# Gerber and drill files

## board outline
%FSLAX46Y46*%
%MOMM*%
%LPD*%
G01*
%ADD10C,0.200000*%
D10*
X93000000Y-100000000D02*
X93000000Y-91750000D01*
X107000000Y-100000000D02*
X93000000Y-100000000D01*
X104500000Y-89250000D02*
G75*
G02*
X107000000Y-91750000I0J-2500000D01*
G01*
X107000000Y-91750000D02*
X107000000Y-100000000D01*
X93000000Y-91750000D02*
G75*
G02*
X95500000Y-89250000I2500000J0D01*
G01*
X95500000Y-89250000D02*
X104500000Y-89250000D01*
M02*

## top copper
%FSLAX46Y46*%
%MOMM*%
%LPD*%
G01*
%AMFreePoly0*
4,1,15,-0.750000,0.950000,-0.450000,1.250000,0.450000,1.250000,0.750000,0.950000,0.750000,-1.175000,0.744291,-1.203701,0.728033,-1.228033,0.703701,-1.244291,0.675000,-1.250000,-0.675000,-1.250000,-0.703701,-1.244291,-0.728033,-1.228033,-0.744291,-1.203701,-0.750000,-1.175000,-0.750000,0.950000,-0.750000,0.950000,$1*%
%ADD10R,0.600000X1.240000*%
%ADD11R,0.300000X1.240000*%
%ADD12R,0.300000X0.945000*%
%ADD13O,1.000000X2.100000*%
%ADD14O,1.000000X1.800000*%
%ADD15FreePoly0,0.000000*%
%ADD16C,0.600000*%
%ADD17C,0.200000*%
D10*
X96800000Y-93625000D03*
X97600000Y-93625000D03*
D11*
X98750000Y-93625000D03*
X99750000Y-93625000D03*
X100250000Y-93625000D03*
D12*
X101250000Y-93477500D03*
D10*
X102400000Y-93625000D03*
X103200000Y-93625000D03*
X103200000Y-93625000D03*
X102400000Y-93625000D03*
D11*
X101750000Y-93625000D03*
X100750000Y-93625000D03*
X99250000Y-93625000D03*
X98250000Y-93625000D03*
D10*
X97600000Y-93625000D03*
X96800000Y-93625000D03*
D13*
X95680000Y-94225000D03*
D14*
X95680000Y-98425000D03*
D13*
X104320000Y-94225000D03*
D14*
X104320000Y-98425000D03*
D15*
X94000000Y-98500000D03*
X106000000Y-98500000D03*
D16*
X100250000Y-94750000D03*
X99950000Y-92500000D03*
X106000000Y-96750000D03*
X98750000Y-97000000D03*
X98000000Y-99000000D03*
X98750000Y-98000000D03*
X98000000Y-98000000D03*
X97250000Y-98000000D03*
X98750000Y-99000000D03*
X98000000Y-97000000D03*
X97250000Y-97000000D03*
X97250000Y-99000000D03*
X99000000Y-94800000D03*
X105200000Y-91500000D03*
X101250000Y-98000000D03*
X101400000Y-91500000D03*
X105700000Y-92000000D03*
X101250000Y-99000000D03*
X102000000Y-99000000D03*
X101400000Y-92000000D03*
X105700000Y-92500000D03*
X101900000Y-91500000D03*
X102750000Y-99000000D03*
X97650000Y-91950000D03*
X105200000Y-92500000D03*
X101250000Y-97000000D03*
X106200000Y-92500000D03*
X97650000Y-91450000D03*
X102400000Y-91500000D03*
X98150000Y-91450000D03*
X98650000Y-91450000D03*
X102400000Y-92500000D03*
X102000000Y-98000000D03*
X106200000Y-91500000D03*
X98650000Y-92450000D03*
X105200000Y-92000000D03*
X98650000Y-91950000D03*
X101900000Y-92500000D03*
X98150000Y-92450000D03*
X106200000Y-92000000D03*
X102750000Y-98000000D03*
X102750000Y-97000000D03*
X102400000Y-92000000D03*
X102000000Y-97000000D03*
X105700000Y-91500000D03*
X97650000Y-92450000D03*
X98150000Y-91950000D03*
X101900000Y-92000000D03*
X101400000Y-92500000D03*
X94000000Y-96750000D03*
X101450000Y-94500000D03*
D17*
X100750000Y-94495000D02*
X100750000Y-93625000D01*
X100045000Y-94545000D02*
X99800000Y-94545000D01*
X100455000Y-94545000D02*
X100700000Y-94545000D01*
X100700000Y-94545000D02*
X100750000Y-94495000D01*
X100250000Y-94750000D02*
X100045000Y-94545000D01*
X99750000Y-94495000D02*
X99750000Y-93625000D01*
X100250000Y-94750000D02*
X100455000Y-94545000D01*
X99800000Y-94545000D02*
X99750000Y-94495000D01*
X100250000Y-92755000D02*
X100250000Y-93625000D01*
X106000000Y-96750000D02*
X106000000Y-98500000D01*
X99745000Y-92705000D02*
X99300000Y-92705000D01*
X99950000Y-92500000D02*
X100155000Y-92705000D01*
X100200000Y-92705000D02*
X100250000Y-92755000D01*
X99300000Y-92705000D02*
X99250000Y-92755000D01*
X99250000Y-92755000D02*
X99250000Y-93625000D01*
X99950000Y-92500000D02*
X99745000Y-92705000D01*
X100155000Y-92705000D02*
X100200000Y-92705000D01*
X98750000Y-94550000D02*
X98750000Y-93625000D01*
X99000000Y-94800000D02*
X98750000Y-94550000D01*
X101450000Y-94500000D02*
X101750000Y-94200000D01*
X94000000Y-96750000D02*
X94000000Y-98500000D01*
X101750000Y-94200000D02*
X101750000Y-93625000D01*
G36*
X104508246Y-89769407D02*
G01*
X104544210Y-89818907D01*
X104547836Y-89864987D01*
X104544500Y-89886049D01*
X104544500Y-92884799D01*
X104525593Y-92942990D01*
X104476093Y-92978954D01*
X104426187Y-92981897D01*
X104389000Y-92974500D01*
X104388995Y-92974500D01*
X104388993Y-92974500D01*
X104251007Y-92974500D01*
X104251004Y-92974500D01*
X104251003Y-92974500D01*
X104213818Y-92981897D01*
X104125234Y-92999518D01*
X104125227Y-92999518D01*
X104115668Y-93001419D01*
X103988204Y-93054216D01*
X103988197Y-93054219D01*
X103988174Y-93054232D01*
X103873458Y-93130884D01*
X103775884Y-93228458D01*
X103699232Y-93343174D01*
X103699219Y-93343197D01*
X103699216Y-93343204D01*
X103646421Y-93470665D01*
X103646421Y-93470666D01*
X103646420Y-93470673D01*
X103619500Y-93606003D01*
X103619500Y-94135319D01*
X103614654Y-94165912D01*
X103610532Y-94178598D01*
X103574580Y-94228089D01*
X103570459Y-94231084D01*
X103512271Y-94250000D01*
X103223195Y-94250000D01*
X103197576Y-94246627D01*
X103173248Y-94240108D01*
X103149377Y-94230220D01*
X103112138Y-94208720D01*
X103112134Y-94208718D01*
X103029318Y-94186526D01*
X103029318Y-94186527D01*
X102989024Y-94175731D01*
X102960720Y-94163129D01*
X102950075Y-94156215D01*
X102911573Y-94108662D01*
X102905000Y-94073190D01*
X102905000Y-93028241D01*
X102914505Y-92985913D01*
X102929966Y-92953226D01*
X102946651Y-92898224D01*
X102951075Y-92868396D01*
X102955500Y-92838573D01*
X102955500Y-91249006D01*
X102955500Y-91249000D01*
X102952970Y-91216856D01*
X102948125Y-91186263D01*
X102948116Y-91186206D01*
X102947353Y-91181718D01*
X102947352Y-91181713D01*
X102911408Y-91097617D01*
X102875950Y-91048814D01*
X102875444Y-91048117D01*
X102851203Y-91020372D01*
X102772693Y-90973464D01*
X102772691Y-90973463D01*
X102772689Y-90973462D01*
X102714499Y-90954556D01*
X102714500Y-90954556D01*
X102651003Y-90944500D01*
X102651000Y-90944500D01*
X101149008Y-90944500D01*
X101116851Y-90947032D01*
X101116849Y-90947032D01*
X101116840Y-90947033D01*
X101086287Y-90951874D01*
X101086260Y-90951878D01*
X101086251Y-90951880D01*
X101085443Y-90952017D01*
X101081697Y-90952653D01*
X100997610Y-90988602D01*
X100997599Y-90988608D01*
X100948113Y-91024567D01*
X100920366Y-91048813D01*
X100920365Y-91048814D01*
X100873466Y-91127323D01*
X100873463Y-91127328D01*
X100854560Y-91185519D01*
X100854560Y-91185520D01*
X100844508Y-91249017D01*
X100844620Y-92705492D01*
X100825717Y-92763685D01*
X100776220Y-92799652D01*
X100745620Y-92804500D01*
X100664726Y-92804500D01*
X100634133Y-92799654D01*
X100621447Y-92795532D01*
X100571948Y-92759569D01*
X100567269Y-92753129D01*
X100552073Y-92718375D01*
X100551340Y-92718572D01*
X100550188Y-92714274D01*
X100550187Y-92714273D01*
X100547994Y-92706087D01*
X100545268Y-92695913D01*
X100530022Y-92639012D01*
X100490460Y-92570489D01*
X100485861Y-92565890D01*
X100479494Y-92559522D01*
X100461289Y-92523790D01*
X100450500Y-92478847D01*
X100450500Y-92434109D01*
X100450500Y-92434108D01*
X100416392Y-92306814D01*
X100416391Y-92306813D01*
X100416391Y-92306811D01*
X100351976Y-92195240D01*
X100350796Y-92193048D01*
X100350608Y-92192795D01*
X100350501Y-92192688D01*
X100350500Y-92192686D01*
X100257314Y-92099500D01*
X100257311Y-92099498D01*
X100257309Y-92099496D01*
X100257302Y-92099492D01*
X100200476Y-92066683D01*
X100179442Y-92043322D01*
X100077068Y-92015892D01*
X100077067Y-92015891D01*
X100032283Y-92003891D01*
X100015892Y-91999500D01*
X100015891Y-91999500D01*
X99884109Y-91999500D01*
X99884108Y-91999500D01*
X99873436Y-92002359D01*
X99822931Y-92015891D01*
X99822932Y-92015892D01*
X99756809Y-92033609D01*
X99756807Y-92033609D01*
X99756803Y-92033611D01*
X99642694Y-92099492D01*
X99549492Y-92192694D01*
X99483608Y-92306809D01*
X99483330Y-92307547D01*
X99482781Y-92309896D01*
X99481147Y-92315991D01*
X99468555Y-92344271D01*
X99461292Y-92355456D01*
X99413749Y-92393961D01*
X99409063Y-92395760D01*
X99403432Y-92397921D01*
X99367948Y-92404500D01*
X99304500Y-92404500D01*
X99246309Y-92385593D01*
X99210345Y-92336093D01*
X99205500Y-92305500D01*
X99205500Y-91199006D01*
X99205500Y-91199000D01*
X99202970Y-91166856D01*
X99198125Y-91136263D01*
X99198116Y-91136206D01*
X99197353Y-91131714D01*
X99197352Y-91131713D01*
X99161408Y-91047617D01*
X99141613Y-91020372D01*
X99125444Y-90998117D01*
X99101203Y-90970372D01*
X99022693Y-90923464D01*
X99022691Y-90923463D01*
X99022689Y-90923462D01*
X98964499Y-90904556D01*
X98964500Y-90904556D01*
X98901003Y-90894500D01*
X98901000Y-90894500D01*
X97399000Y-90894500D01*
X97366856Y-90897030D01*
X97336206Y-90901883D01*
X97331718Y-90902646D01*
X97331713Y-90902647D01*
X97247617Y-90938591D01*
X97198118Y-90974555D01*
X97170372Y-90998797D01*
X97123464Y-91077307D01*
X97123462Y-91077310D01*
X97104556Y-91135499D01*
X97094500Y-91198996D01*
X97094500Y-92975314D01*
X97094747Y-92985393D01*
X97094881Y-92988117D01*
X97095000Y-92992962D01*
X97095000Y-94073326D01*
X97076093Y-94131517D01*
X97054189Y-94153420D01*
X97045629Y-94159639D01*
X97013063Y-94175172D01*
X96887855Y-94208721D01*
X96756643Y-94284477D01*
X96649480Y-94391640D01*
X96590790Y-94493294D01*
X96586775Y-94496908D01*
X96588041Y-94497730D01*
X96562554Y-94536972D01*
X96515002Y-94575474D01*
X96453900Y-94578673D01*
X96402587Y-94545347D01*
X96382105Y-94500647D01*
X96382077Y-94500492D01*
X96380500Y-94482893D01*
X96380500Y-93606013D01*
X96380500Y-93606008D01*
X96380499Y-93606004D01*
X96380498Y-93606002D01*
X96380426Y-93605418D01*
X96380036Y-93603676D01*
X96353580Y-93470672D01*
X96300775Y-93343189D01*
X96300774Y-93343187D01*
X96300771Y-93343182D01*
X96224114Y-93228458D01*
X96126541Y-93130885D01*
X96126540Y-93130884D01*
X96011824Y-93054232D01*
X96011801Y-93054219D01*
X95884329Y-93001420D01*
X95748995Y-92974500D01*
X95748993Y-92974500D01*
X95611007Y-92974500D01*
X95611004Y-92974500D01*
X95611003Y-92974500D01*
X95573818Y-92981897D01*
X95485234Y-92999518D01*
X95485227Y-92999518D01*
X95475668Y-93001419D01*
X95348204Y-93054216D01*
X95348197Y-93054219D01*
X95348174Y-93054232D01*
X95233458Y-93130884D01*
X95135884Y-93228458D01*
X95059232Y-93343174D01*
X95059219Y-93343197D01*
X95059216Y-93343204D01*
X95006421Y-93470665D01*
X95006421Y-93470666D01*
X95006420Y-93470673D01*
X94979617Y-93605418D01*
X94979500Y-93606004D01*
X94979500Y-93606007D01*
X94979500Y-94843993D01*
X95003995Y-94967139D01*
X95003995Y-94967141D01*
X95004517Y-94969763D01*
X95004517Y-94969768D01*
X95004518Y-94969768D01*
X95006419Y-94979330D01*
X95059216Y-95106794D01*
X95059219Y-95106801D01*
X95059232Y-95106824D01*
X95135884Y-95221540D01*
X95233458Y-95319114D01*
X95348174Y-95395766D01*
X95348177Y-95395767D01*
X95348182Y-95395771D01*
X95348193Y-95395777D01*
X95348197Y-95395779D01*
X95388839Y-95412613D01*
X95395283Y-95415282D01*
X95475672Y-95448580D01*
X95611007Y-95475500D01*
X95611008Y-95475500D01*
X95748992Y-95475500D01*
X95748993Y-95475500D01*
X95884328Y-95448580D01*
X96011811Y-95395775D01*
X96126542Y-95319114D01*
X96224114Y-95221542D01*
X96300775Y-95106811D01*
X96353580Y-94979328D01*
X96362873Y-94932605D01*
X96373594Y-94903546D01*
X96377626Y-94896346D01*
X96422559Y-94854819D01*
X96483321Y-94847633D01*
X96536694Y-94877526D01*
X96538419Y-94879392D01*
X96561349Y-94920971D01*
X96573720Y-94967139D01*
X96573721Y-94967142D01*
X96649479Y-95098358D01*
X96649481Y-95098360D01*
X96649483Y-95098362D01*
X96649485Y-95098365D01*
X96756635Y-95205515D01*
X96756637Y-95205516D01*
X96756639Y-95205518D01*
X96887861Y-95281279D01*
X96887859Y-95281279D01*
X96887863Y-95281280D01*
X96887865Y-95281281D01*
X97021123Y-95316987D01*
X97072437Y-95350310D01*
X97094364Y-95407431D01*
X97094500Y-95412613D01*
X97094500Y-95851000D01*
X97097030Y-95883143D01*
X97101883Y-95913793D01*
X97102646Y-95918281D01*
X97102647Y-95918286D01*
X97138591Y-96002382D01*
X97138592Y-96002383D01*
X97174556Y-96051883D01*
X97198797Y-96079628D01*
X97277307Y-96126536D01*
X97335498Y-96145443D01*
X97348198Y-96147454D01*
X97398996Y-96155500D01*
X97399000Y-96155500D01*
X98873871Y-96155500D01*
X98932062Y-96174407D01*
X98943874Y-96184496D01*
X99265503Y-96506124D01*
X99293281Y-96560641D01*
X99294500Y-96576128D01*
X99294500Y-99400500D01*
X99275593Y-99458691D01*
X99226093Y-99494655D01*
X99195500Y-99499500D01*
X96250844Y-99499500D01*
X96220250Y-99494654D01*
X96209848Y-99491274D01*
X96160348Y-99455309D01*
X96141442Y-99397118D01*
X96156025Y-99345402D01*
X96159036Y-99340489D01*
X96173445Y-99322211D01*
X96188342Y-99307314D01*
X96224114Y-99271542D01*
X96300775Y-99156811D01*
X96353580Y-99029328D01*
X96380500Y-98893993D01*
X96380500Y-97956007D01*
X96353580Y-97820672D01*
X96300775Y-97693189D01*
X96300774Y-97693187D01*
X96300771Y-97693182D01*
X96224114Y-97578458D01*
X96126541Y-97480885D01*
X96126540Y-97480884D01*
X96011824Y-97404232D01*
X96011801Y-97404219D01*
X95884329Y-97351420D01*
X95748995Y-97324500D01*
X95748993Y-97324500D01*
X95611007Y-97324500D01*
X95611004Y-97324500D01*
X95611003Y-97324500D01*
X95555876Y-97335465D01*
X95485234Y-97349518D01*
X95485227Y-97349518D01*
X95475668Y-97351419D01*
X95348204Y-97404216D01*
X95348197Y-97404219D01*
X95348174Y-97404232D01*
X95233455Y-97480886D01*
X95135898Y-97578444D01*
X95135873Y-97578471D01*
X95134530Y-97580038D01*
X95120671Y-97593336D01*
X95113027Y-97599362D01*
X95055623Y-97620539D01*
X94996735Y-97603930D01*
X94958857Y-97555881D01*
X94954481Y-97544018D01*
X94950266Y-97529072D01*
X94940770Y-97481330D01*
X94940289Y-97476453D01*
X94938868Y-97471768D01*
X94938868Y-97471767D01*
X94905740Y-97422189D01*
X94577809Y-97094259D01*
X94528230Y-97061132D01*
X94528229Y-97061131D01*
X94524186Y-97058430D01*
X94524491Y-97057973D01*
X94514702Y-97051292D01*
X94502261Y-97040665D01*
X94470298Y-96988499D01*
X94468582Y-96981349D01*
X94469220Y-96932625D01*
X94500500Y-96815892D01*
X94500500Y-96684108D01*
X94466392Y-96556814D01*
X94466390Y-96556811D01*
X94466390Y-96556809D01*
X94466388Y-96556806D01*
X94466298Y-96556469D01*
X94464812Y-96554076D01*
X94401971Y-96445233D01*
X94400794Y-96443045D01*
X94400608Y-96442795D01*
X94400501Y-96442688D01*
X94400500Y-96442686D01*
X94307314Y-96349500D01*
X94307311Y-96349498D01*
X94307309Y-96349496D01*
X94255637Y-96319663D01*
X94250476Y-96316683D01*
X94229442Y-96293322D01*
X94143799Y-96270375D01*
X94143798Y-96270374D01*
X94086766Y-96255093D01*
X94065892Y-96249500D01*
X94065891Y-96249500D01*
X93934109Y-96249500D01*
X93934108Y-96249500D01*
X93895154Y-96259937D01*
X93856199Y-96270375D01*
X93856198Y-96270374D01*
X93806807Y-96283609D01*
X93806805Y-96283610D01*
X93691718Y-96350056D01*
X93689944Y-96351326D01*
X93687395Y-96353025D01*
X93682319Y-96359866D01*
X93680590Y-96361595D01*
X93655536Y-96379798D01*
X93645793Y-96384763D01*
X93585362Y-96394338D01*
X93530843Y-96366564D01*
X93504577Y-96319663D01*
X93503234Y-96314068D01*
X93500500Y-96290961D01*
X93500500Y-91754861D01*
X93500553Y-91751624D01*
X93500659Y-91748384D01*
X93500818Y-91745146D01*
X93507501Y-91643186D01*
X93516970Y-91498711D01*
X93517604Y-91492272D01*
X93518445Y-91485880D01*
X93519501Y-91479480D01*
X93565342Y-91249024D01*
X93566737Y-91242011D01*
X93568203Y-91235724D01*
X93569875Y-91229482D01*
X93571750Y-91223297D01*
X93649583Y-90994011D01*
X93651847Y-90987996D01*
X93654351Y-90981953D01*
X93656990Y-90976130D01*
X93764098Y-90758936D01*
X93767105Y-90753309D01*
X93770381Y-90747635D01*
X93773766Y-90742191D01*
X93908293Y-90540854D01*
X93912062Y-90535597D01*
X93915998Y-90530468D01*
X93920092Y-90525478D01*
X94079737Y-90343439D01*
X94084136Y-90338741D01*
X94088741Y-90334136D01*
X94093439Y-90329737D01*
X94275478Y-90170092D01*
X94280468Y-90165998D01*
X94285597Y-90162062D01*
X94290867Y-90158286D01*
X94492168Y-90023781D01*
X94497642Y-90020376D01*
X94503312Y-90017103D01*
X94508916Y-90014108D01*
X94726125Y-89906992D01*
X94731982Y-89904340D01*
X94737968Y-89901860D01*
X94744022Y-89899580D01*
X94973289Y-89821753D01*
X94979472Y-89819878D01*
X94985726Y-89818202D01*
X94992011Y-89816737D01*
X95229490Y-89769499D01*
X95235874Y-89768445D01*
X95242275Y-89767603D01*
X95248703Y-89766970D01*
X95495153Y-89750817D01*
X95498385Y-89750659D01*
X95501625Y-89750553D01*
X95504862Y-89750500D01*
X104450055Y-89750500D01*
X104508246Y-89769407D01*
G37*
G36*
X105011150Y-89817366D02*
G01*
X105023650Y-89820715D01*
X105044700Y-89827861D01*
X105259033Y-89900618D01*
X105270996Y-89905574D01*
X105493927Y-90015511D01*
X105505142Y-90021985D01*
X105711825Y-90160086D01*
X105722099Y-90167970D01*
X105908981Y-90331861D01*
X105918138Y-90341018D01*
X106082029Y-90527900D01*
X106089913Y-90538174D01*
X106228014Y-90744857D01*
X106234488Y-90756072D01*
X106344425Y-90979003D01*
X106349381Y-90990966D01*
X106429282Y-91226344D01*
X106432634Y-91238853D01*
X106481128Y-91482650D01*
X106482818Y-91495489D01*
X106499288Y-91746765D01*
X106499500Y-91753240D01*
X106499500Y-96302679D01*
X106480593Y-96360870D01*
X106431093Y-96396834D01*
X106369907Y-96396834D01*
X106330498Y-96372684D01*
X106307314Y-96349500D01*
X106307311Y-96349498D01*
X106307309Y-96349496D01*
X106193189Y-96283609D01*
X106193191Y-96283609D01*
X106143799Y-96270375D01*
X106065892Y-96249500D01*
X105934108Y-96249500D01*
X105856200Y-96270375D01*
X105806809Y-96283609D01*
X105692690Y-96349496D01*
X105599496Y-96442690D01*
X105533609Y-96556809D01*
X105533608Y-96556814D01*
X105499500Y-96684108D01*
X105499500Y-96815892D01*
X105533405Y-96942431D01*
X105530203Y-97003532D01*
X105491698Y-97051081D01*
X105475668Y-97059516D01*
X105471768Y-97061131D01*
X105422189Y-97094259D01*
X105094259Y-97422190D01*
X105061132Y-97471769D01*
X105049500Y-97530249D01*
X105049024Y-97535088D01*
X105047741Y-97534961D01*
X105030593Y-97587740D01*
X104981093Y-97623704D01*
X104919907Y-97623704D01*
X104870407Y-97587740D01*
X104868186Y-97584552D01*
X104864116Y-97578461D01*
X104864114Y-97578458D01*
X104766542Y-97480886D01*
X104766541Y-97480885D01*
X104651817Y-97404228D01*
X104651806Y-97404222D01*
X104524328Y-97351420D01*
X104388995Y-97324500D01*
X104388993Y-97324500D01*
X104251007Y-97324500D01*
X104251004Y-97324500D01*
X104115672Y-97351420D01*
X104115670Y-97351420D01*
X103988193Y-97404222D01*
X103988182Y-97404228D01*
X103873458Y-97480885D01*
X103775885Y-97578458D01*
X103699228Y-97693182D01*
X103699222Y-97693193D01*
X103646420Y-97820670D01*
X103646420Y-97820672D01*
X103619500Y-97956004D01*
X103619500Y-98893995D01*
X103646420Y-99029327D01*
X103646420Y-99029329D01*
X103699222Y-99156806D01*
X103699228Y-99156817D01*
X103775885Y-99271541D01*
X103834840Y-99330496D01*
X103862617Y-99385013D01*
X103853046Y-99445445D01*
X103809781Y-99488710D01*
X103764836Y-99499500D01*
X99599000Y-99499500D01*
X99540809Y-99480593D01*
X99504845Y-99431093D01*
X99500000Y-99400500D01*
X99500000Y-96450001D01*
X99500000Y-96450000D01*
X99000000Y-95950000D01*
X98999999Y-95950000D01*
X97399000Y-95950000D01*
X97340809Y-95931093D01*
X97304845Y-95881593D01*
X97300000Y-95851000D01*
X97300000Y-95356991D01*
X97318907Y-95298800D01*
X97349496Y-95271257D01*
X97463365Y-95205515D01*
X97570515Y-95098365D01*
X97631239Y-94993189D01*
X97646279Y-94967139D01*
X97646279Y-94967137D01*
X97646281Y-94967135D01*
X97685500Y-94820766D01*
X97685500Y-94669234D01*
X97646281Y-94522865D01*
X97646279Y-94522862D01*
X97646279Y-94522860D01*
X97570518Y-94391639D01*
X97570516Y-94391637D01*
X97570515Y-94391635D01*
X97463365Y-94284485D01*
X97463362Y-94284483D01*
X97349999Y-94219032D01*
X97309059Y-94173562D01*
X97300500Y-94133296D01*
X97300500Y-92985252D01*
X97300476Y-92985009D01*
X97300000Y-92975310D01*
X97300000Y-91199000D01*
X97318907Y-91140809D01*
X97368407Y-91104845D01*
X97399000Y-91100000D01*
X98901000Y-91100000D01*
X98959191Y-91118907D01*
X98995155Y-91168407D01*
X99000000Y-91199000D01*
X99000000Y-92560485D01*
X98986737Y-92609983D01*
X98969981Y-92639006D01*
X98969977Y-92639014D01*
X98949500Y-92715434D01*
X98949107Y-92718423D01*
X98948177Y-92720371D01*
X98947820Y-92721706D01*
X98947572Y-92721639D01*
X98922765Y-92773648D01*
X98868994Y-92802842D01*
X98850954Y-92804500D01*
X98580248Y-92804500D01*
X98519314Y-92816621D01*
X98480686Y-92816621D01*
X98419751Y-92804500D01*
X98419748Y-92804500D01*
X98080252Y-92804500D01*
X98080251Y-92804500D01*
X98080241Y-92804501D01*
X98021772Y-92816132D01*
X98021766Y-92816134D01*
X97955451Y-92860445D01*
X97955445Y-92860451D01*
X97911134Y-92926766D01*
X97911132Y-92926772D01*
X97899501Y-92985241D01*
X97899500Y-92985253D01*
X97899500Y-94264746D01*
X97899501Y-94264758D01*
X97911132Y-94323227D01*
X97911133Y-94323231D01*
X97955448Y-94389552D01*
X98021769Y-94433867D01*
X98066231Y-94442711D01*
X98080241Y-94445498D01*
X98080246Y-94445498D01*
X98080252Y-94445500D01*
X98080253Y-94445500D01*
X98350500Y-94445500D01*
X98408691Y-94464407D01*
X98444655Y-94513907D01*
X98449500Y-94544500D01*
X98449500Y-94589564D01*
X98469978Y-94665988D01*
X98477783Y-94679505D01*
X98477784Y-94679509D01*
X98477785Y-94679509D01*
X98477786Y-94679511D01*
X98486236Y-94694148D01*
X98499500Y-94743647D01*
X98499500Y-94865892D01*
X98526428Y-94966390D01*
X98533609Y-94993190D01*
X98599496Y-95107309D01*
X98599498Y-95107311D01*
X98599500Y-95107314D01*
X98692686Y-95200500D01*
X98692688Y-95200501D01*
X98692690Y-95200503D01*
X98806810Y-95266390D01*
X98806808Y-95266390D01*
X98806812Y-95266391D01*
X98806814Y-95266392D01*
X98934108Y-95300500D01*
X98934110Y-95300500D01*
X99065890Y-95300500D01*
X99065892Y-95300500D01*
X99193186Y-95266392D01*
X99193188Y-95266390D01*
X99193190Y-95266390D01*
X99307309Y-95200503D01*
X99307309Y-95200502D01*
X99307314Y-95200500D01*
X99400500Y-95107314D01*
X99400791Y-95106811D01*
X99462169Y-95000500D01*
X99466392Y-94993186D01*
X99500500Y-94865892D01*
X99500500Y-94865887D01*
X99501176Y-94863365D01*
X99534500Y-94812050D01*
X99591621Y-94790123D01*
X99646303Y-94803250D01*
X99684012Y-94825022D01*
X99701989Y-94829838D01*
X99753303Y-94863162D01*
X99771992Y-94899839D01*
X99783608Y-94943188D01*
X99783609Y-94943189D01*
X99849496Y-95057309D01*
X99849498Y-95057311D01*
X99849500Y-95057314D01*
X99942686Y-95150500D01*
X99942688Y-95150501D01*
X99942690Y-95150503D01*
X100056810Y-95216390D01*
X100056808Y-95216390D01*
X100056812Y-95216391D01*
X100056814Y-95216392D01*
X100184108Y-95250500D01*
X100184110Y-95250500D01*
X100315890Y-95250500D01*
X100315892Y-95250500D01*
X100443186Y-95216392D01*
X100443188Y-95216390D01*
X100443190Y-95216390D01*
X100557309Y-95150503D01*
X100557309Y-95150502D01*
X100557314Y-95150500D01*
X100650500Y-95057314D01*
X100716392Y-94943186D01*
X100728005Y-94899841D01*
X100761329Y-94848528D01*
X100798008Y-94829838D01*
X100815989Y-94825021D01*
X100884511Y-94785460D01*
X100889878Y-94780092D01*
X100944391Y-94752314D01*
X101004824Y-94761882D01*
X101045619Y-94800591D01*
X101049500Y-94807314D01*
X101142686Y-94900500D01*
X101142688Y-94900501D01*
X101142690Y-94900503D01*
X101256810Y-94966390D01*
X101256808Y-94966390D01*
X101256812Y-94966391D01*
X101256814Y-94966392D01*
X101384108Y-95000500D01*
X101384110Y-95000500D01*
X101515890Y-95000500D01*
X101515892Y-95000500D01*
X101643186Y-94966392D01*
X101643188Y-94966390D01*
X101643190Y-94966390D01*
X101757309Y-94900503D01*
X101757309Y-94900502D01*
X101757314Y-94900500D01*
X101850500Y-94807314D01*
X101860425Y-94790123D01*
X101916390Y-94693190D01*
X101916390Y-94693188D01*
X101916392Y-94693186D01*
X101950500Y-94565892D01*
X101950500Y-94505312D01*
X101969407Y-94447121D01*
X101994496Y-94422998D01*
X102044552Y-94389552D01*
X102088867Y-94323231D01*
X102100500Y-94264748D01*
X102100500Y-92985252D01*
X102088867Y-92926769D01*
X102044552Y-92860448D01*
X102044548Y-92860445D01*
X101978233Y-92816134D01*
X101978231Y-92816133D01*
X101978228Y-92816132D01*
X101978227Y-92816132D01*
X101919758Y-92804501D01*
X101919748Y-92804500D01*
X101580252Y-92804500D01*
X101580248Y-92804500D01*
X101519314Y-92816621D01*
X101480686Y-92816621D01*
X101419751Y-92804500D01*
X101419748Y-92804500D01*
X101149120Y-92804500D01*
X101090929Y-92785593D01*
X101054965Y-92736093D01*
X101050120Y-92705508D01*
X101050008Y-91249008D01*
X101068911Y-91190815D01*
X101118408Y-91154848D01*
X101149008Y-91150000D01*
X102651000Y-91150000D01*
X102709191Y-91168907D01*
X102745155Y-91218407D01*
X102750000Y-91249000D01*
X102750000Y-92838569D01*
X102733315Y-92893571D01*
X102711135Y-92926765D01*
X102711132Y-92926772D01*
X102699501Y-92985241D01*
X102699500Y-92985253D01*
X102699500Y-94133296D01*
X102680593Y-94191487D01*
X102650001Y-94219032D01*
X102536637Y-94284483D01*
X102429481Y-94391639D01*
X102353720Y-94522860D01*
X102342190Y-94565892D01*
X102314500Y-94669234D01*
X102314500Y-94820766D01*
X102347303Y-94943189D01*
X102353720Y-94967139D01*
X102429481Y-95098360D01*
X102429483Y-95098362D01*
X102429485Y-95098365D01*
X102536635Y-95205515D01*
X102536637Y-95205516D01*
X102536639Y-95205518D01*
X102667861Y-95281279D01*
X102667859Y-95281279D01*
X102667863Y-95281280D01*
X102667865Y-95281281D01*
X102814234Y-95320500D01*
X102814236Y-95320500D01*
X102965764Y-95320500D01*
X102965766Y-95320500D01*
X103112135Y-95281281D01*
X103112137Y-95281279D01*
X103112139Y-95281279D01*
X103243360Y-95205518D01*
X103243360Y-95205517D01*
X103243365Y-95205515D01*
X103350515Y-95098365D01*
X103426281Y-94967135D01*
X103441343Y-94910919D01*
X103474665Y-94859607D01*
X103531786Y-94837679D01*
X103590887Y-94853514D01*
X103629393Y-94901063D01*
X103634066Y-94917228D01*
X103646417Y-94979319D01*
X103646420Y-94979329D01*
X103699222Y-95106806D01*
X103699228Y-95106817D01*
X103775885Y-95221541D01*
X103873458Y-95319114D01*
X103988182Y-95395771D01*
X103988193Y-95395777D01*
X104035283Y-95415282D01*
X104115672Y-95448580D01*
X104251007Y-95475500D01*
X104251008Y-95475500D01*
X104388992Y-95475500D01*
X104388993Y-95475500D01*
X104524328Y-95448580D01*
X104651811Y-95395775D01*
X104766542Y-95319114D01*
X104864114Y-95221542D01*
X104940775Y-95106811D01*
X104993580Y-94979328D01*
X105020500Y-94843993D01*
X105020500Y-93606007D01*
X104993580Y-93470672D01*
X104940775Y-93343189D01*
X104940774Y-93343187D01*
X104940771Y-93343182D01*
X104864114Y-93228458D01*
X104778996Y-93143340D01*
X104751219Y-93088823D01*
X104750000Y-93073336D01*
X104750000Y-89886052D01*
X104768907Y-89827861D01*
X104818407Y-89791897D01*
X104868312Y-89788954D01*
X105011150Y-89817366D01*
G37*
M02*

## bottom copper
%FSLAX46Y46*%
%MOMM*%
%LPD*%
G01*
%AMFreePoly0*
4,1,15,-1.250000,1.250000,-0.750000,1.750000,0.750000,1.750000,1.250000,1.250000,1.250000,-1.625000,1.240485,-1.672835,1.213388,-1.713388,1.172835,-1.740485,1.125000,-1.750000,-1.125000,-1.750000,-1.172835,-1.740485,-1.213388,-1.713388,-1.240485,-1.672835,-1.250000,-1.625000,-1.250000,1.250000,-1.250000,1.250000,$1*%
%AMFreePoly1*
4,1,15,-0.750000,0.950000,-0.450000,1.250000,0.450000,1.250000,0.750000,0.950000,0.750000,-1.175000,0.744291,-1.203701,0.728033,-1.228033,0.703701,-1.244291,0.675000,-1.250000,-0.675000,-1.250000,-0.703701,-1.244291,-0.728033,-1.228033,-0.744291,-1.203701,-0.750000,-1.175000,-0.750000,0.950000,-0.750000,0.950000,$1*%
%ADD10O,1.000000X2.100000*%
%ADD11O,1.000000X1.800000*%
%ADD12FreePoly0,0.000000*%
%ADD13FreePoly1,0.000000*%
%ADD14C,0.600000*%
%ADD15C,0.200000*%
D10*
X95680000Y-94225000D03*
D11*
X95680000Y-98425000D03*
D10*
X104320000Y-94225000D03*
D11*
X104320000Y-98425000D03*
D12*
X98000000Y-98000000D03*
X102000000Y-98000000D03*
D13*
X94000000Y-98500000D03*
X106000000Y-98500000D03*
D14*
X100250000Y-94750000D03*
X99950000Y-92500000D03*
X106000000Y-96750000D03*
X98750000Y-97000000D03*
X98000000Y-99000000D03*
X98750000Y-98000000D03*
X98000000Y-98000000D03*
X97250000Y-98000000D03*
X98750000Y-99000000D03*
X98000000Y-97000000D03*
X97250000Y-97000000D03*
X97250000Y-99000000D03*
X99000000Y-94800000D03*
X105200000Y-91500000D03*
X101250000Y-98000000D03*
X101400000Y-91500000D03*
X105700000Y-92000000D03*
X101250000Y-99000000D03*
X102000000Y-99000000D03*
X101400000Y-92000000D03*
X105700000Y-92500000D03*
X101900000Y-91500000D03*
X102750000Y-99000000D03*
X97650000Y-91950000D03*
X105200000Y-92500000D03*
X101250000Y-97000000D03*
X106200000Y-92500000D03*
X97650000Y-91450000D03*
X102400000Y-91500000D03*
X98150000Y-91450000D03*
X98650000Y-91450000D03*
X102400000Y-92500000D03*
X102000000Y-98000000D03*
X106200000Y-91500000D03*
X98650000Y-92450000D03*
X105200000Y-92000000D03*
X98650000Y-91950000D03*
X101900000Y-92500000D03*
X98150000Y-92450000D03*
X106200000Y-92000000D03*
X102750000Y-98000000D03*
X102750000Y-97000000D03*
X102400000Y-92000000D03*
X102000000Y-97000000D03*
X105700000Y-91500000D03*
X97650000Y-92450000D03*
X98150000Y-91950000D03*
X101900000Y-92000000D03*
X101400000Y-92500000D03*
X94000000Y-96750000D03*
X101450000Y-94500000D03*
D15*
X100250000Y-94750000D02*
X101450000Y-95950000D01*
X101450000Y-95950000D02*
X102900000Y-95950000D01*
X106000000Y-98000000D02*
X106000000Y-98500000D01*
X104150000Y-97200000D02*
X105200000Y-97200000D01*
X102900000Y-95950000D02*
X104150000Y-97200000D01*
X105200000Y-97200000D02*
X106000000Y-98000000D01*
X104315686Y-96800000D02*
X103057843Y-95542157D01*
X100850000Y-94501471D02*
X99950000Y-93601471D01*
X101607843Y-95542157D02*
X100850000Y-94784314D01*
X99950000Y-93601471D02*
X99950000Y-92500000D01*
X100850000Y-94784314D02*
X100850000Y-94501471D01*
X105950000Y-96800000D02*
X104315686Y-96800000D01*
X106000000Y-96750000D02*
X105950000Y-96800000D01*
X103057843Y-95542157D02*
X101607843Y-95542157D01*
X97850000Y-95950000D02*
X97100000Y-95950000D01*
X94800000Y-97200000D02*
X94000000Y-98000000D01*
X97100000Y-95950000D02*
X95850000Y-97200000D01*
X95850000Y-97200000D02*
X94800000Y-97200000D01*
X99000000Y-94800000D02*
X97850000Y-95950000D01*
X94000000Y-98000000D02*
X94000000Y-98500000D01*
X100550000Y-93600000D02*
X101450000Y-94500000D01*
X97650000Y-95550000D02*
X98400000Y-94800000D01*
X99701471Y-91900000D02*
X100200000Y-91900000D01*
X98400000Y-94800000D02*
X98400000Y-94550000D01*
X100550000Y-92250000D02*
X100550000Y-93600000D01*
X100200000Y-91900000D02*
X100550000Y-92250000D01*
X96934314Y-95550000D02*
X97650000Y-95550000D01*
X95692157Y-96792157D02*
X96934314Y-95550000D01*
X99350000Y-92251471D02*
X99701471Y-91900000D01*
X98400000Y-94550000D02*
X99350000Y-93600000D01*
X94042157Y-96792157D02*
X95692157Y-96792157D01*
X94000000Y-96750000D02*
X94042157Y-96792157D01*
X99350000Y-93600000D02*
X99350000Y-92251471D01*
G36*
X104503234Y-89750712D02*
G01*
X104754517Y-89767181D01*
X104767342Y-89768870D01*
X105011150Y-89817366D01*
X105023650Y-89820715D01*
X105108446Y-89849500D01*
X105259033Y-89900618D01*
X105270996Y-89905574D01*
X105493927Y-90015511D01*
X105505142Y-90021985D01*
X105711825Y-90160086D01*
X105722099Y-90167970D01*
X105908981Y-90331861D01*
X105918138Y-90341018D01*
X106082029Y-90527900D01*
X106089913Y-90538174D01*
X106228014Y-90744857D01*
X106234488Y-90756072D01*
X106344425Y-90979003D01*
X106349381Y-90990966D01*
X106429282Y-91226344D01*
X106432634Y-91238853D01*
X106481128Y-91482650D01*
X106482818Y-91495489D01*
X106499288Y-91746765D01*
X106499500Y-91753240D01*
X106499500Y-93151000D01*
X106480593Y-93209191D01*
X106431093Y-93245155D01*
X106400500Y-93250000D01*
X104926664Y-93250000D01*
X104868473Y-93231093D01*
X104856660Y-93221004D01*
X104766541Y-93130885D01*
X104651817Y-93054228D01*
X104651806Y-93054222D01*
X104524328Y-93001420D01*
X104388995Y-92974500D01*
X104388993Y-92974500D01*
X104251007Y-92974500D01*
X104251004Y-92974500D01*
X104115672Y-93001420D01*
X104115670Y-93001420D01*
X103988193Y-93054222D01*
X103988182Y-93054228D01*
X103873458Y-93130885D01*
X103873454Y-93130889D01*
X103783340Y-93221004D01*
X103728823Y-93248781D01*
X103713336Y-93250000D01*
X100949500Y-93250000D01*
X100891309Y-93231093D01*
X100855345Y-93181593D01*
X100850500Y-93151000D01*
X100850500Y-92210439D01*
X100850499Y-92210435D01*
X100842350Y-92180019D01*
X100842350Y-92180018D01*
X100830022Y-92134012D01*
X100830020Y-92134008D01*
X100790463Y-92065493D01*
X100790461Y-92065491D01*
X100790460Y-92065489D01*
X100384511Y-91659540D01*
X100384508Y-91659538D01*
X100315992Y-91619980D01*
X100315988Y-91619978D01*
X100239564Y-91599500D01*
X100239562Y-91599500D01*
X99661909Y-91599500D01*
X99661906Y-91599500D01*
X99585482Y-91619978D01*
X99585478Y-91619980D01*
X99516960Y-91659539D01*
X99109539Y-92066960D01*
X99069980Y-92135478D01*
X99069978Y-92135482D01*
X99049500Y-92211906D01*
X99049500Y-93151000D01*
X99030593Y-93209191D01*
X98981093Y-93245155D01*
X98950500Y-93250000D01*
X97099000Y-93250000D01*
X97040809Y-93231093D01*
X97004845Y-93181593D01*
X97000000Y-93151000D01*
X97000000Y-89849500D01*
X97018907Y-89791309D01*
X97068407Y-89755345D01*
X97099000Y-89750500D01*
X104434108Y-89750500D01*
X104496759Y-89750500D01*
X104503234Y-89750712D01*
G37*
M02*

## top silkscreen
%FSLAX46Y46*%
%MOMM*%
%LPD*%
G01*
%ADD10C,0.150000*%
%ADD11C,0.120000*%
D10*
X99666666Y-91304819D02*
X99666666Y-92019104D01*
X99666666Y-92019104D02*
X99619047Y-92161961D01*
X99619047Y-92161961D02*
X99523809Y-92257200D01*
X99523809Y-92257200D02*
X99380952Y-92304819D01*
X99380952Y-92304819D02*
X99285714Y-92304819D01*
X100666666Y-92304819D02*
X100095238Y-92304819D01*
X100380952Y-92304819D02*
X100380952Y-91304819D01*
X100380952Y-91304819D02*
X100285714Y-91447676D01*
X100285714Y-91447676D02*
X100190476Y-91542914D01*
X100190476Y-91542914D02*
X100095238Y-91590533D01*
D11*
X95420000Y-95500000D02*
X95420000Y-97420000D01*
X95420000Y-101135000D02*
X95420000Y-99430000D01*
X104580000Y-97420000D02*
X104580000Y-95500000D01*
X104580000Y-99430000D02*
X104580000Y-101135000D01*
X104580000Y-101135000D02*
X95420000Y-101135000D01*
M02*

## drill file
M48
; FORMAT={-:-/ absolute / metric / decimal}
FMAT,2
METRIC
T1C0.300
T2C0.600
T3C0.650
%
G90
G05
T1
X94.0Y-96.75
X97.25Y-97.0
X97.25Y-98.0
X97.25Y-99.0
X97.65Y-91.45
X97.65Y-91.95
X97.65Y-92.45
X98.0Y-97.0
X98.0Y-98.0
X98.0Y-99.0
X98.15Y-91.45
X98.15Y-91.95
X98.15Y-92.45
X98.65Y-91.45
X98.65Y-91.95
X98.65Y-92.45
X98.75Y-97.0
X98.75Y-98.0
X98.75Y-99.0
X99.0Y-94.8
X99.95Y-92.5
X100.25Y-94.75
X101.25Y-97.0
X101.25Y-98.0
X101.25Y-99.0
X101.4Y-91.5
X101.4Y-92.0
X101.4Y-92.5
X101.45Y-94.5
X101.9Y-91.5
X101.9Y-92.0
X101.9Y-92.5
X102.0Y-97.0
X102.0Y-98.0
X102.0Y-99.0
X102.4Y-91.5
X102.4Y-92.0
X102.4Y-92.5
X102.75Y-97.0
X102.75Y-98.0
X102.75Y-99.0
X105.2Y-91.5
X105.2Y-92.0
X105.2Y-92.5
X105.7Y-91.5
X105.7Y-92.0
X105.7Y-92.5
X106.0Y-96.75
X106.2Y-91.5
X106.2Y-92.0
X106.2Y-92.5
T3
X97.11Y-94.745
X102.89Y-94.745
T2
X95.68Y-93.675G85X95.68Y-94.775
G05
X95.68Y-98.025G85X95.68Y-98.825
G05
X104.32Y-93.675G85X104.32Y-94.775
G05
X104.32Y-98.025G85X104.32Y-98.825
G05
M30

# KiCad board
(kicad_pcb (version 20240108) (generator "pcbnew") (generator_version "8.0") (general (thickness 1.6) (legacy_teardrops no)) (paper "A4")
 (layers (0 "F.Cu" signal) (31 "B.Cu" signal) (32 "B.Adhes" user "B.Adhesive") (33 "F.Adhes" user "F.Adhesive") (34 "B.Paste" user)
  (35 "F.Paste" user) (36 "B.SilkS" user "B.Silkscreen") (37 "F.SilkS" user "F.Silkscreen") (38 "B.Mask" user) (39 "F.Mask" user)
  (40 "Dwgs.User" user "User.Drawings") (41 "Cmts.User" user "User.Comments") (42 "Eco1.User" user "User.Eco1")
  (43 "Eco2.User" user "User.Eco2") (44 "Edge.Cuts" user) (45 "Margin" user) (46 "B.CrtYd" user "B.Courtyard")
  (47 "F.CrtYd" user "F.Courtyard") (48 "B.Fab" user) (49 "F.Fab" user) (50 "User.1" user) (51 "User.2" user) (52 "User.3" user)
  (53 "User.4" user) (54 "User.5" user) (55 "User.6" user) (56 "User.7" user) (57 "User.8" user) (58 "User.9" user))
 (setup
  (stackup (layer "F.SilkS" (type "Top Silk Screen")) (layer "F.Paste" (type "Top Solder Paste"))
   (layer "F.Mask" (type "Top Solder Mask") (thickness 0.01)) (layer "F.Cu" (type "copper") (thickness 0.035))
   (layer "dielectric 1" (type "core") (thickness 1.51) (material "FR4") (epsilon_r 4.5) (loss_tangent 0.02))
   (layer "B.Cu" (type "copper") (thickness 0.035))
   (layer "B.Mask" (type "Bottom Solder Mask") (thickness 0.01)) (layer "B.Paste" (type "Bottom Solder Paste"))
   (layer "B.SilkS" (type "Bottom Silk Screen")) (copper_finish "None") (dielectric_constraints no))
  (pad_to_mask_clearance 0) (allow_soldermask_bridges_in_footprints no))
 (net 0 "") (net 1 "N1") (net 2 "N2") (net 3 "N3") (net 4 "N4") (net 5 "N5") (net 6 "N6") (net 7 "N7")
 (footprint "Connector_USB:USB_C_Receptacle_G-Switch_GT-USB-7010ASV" (layer "F.Cu") (at 100 97.35)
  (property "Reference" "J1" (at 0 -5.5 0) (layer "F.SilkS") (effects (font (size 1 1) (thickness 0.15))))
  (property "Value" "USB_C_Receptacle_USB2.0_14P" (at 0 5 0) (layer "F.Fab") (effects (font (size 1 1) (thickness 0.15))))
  (fp_line (start -4.58 -1.85) (end -4.58 0.07) (stroke (width 0.12) (type solid)) (layer "F.SilkS"))
  (fp_line (start -4.58 3.785) (end -4.58 2.08) (stroke (width 0.12) (type solid)) (layer "F.SilkS"))
  (fp_line (start 4.58 0.07) (end 4.58 -1.85) (stroke (width 0.12) (type solid)) (layer "F.SilkS"))
  (fp_line (start 4.58 2.08) (end 4.58 3.785) (stroke (width 0.12) (type solid)) (layer "F.SilkS"))
  (fp_line (start 4.58 3.785) (end -4.58 3.785) (stroke (width 0.12) (type solid)) (layer "F.SilkS"))
  (pad "" np_thru_hole circle (at -2.89 -2.605) (size 0.65 0.65) (drill 0.65) (layers "*.Cu" "*.Mask"))
  (pad "" np_thru_hole circle (at 2.89 -2.605) (size 0.65 0.65) (drill 0.65) (layers "*.Cu" "*.Mask"))
  (pad "A1" smd rect (at -3.2 -3.725) (size 0.6 1.24) (layers "F.Cu" "F.Paste" "F.Mask") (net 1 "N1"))
  (pad "A4" smd rect (at -2.4 -3.725) (size 0.6 1.24) (layers "F.Cu" "F.Paste" "F.Mask") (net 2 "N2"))
  (pad "A5" smd rect (at -1.25 -3.725) (size 0.3 1.24) (layers "F.Cu" "F.Paste" "F.Mask") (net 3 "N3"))
  (pad "A6" smd rect (at -0.25 -3.725) (size 0.3 1.24) (layers "F.Cu" "F.Paste" "F.Mask") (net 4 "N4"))
  (pad "A7" smd rect (at 0.25 -3.725) (size 0.3 1.24) (layers "F.Cu" "F.Paste" "F.Mask") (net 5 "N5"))
  (pad "A8" smd rect (at 1.25 -3.8725) (size 0.3 0.945) (layers "F.Cu" "F.Paste" "F.Mask"))
  (pad "A9" smd rect (at 2.4 -3.725) (size 0.6 1.24) (layers "F.Cu" "F.Paste" "F.Mask") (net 2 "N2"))
  (pad "A12" smd rect (at 3.2 -3.725) (size 0.6 1.24) (layers "F.Cu" "F.Paste" "F.Mask") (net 1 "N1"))
  (pad "B1" smd rect (at 3.2 -3.725) (size 0.6 1.24) (layers "F.Cu" "F.Paste" "F.Mask") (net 1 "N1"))
  (pad "B4" smd rect (at 2.4 -3.725) (size 0.6 1.24) (layers "F.Cu" "F.Paste" "F.Mask") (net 2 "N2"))
  (pad "B5" smd rect (at 1.75 -3.725) (size 0.3 1.24) (layers "F.Cu" "F.Paste" "F.Mask") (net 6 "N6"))
  (pad "B6" smd rect (at 0.75 -3.725) (size 0.3 1.24) (layers "F.Cu" "F.Paste" "F.Mask") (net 4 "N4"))
  (pad "B7" smd rect (at -0.75 -3.725) (size 0.3 1.24) (layers "F.Cu" "F.Paste" "F.Mask") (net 5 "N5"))
  (pad "B8" smd rect (at -1.75 -3.725) (size 0.3 1.24) (layers "F.Cu" "F.Paste" "F.Mask"))
  (pad "B9" smd rect (at -2.4 -3.725) (size 0.6 1.24) (layers "F.Cu" "F.Paste" "F.Mask") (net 2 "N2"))
  (pad "B12" smd rect (at -3.2 -3.725) (size 0.6 1.24) (layers "F.Cu" "F.Paste" "F.Mask") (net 1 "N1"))
  (pad "S1" thru_hole oval (at -4.32 -3.125) (size 1 2.1) (drill oval 0.6 1.7) (layers "*.Cu" "*.Mask") (remove_unused_layers no)
   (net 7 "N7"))
  (pad "S1" thru_hole oval (at -4.32 1.075) (size 1 1.8) (drill oval 0.6 1.4) (layers "*.Cu" "*.Mask") (remove_unused_layers no)
   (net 7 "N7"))
  (pad "S1" thru_hole oval (at 4.32 -3.125) (size 1 2.1) (drill oval 0.6 1.7) (layers "*.Cu" "*.Mask") (remove_unused_layers no)
   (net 7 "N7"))
  (pad "S1" thru_hole oval (at 4.32 1.075) (size 1 1.8) (drill oval 0.6 1.4) (layers "*.Cu" "*.Mask") (remove_unused_layers no) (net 7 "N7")))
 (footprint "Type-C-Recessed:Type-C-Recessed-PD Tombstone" (layer "F.Cu") (at 100 100)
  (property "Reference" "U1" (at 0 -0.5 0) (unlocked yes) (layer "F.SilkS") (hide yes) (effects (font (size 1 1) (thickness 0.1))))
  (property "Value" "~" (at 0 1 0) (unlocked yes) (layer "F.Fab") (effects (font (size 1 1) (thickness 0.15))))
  (pad "1" smd roundrect (at -2 -2) (size 2.5 3.5) (layers "B.Cu" "B.Mask") (roundrect_rratio 0.05) (chamfer_ratio 0.2)
   (chamfer top_left top_right) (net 1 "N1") (thermal_bridge_angle 45))
  (pad "2" smd roundrect (at 2 -2) (size 2.5 3.5) (layers "B.Cu" "B.Mask") (roundrect_rratio 0.05) (chamfer_ratio 0.2)
   (chamfer top_left top_right) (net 2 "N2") (thermal_bridge_angle 45))
  (pad "3" smd roundrect (at -6 -1.5) (size 1.5 2.5) (layers "B.Cu" "B.Mask") (roundrect_rratio 0.05) (chamfer_ratio 0.2)
   (chamfer top_left top_right) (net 3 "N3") (thermal_bridge_angle 45))
  (pad "4" smd roundrect (at -6 -1.5) (size 1.5 2.5) (layers "F.Cu" "F.Mask") (roundrect_rratio 0.05) (chamfer_ratio 0.2)
   (chamfer top_left top_right) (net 6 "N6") (thermal_bridge_angle 45))
  (pad "5" smd roundrect (at 6 -1.5) (size 1.5 2.5) (layers "B.Cu" "B.Mask") (roundrect_rratio 0.05) (chamfer_ratio 0.2)
   (chamfer top_left top_right) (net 4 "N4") (thermal_bridge_angle 45))
  (pad "6" smd roundrect (at 6 -1.5) (size 1.5 2.5) (layers "F.Cu" "F.Mask") (roundrect_rratio 0.05) (chamfer_ratio 0.2)
   (chamfer top_left top_right) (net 5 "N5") (thermal_bridge_angle 45)))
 (gr_line (start 93 100) (end 93 91.75) (stroke (width 0.2) (type default)) (layer "Edge.Cuts"))
 (gr_line (start 107 100) (end 93 100) (stroke (width 0.2) (type default)) (layer "Edge.Cuts"))
 (gr_arc (start 104.5 89.25) (mid 106.267767 89.982233) (end 107 91.75) (stroke (width 0.2) (type default)) (layer "Edge.Cuts"))
 (gr_line (start 107 91.75) (end 107 100) (stroke (width 0.2) (type default)) (layer "Edge.Cuts"))
 (gr_arc (start 93 91.75) (mid 93.732233 89.982233) (end 95.5 89.25) (stroke (width 0.2) (type default)) (layer "Edge.Cuts"))
 (gr_line (start 95.5 89.25) (end 104.5 89.25) (stroke (width 0.2) (type default)) (layer "Edge.Cuts"))
 (segment (start 100.75 94.495) (end 100.75 93.625) (width 0.2) (layer "F.Cu") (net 4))
 (segment (start 100.045 94.545) (end 99.8 94.545) (width 0.2) (layer "F.Cu") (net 4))
 (segment (start 100.455 94.545) (end 100.7 94.545) (width 0.2) (layer "F.Cu") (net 4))
 (segment (start 100.7 94.545) (end 100.75 94.495) (width 0.2) (layer "F.Cu") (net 4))
 (segment (start 100.25 94.75) (end 100.045 94.545) (width 0.2) (layer "F.Cu") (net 4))
 (segment (start 99.75 94.495) (end 99.75 93.625) (width 0.2) (layer "F.Cu") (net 4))
 (segment (start 100.25 94.75) (end 100.455 94.545) (width 0.2) (layer "F.Cu") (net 4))
 (segment (start 99.8 94.545) (end 99.75 94.495) (width 0.2) (layer "F.Cu") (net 4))
 (via (at 100.25 94.75) (size 0.6) (drill 0.3) (layers "F.Cu" "B.Cu") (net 4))
 (segment (start 100.25 94.75) (end 101.45 95.95) (width 0.2) (layer "B.Cu") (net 4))
 (segment (start 101.45 95.95) (end 102.9 95.95) (width 0.2) (layer "B.Cu") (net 4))
 (segment (start 106 98) (end 106 98.5) (width 0.2) (layer "B.Cu") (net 4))
 (segment (start 104.15 97.2) (end 105.2 97.2) (width 0.2) (layer "B.Cu") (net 4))
 (segment (start 102.9 95.95) (end 104.15 97.2) (width 0.2) (layer "B.Cu") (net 4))
 (segment (start 105.2 97.2) (end 106 98) (width 0.2) (layer "B.Cu") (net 4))
 (segment (start 100.25 92.755) (end 100.25 93.625) (width 0.2) (layer "F.Cu") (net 5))
 (segment (start 106 96.75) (end 106 98.5) (width 0.2) (layer "F.Cu") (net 5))
 (segment (start 99.745 92.705) (end 99.3 92.705) (width 0.2) (layer "F.Cu") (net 5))
 (segment (start 99.95 92.5) (end 100.155 92.705) (width 0.2) (layer "F.Cu") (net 5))
 (segment (start 100.2 92.705) (end 100.25 92.755) (width 0.2) (layer "F.Cu") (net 5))
 (segment (start 99.3 92.705) (end 99.25 92.755) (width 0.2) (layer "F.Cu") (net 5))
 (segment (start 99.25 92.755) (end 99.25 93.625) (width 0.2) (layer "F.Cu") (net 5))
 (segment (start 99.95 92.5) (end 99.745 92.705) (width 0.2) (layer "F.Cu") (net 5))
 (segment (start 100.155 92.705) (end 100.2 92.705) (width 0.2) (layer "F.Cu") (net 5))
 (via (at 99.95 92.5) (size 0.6) (drill 0.3) (layers "F.Cu" "B.Cu") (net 5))
 (via (at 106 96.75) (size 0.6) (drill 0.3) (layers "F.Cu" "B.Cu") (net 5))
 (segment (start 104.315686 96.8) (end 103.057843 95.542157) (width 0.2) (layer "B.Cu") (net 5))
 (segment (start 100.85 94.501471) (end 99.95 93.601471) (width 0.2) (layer "B.Cu") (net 5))
 (segment (start 101.607843 95.542157) (end 100.85 94.784314) (width 0.2) (layer "B.Cu") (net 5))
 (segment (start 99.95 93.601471) (end 99.95 92.5) (width 0.2) (layer "B.Cu") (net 5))
 (segment (start 100.85 94.784314) (end 100.85 94.501471) (width 0.2) (layer "B.Cu") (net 5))
 (segment (start 105.95 96.8) (end 104.315686 96.8) (width 0.2) (layer "B.Cu") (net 5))
 (segment (start 106 96.75) (end 105.95 96.8) (width 0.2) (layer "B.Cu") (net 5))
 (segment (start 103.057843 95.542157) (end 101.607843 95.542157) (width 0.2) (layer "B.Cu") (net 5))
 (via (at 98.75 97) (size 0.6) (drill 0.3) (layers "F.Cu" "B.Cu") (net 1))
 (via (at 98 99) (size 0.6) (drill 0.3) (layers "F.Cu" "B.Cu") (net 1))
 (via (at 98.75 98) (size 0.6) (drill 0.3) (layers "F.Cu" "B.Cu") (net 1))
 (via (at 98 98) (size 0.6) (drill 0.3) (layers "F.Cu" "B.Cu") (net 1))
 (via (at 97.25 98) (size 0.6) (drill 0.3) (layers "F.Cu" "B.Cu") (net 1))
 (via (at 98.75 99) (size 0.6) (drill 0.3) (layers "F.Cu" "B.Cu") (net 1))
 (via (at 98 97) (size 0.6) (drill 0.3) (layers "F.Cu" "B.Cu") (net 1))
 (via (at 97.25 97) (size 0.6) (drill 0.3) (layers "F.Cu" "B.Cu") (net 1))
 (via (at 97.25 99) (size 0.6) (drill 0.3) (layers "F.Cu" "B.Cu") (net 1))
 (segment (start 98.75 94.55) (end 98.75 93.625) (width 0.2) (layer "F.Cu") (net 3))
 (segment (start 99 94.8) (end 98.75 94.55) (width 0.2) (layer "F.Cu") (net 3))
 (via (at 99 94.8) (size 0.6) (drill 0.3) (layers "F.Cu" "B.Cu") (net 3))
 (segment (start 97.85 95.95) (end 97.1 95.95) (width 0.2) (layer "B.Cu") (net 3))
 (segment (start 94.8 97.2) (end 94 98) (width 0.2) (layer "B.Cu") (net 3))
 (segment (start 97.1 95.95) (end 95.85 97.2) (width 0.2) (layer "B.Cu") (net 3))
 (segment (start 95.85 97.2) (end 94.8 97.2) (width 0.2) (layer "B.Cu") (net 3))
 (segment (start 99 94.8) (end 97.85 95.95) (width 0.2) (layer "B.Cu") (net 3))
 (segment (start 94 98) (end 94 98.5) (width 0.2) (layer "B.Cu") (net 3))
 (via (at 105.2 91.5) (size 0.6) (drill 0.3) (layers "F.Cu" "B.Cu") (free yes) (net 2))
 (via (at 101.25 98) (size 0.6) (drill 0.3) (layers "F.Cu" "B.Cu") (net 2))
 (via (at 101.4 91.5) (size 0.6) (drill 0.3) (layers "F.Cu" "B.Cu") (free yes) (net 2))
 (via (at 105.7 92) (size 0.6) (drill 0.3) (layers "F.Cu" "B.Cu") (free yes) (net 2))
 (via (at 101.25 99) (size 0.6) (drill 0.3) (layers "F.Cu" "B.Cu") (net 2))
 (via (at 102 99) (size 0.6) (drill 0.3) (layers "F.Cu" "B.Cu") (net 2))
 (via (at 101.4 92) (size 0.6) (drill 0.3) (layers "F.Cu" "B.Cu") (free yes) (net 2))
 (via (at 105.7 92.5) (size 0.6) (drill 0.3) (layers "F.Cu" "B.Cu") (free yes) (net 2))
 (via (at 101.9 91.5) (size 0.6) (drill 0.3) (layers "F.Cu" "B.Cu") (free yes) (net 2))
 (via (at 102.75 99) (size 0.6) (drill 0.3) (layers "F.Cu" "B.Cu") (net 2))
 (via (at 97.65 91.95) (size 0.6) (drill 0.3) (layers "F.Cu" "B.Cu") (free yes) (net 2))
 (via (at 105.2 92.5) (size 0.6) (drill 0.3) (layers "F.Cu" "B.Cu") (free yes) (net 2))
 (via (at 101.25 97) (size 0.6) (drill 0.3) (layers "F.Cu" "B.Cu") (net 2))
 (via (at 106.2 92.5) (size 0.6) (drill 0.3) (layers "F.Cu" "B.Cu") (free yes) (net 2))
 (via (at 97.65 91.45) (size 0.6) (drill 0.3) (layers "F.Cu" "B.Cu") (free yes) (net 2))
 (via (at 102.4 91.5) (size 0.6) (drill 0.3) (layers "F.Cu" "B.Cu") (free yes) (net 2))
 (via (at 98.15 91.45) (size 0.6) (drill 0.3) (layers "F.Cu" "B.Cu") (free yes) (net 2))
 (via (at 98.65 91.45) (size 0.6) (drill 0.3) (layers "F.Cu" "B.Cu") (free yes) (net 2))
 (via (at 102.4 92.5) (size 0.6) (drill 0.3) (layers "F.Cu" "B.Cu") (free yes) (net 2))
 (via (at 102 98) (size 0.6) (drill 0.3) (layers "F.Cu" "B.Cu") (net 2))
 (via (at 106.2 91.5) (size 0.6) (drill 0.3) (layers "F.Cu" "B.Cu") (free yes) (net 2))
 (via (at 98.65 92.45) (size 0.6) (drill 0.3) (layers "F.Cu" "B.Cu") (free yes) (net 2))
 (via (at 105.2 92) (size 0.6) (drill 0.3) (layers "F.Cu" "B.Cu") (free yes) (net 2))
 (via (at 98.65 91.95) (size 0.6) (drill 0.3) (layers "F.Cu" "B.Cu") (free yes) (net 2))
 (via (at 101.9 92.5) (size 0.6) (drill 0.3) (layers "F.Cu" "B.Cu") (free yes) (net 2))
 (via (at 98.15 92.45) (size 0.6) (drill 0.3) (layers "F.Cu" "B.Cu") (free yes) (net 2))
 (via (at 106.2 92) (size 0.6) (drill 0.3) (layers "F.Cu" "B.Cu") (free yes) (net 2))
 (via (at 102.75 98) (size 0.6) (drill 0.3) (layers "F.Cu" "B.Cu") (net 2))
 (via (at 102.75 97) (size 0.6) (drill 0.3) (layers "F.Cu" "B.Cu") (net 2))
 (via (at 102.4 92) (size 0.6) (drill 0.3) (layers "F.Cu" "B.Cu") (free yes) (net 2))
 (via (at 102 97) (size 0.6) (drill 0.3) (layers "F.Cu" "B.Cu") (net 2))
 (via (at 105.7 91.5) (size 0.6) (drill 0.3) (layers "F.Cu" "B.Cu") (free yes) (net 2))
 (via (at 97.65 92.45) (size 0.6) (drill 0.3) (layers "F.Cu" "B.Cu") (free yes) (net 2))
 (via (at 98.15 91.95) (size 0.6) (drill 0.3) (layers "F.Cu" "B.Cu") (free yes) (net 2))
 (via (at 101.9 92) (size 0.6) (drill 0.3) (layers "F.Cu" "B.Cu") (free yes) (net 2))
 (via (at 101.4 92.5) (size 0.6) (drill 0.3) (layers "F.Cu" "B.Cu") (free yes) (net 2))
 (segment (start 101.45 94.5) (end 101.75 94.2) (width 0.2) (layer "F.Cu") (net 6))
 (segment (start 94 96.75) (end 94 98.5) (width 0.2) (layer "F.Cu") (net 6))
 (segment (start 101.75 94.2) (end 101.75 93.625) (width 0.2) (layer "F.Cu") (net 6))
 (via (at 94 96.75) (size 0.6) (drill 0.3) (layers "F.Cu" "B.Cu") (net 6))
 (via (at 101.45 94.5) (size 0.6) (drill 0.3) (layers "F.Cu" "B.Cu") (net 6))
 (segment (start 100.55 93.6) (end 101.45 94.5) (width 0.2) (layer "B.Cu") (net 6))
 (segment (start 97.65 95.55) (end 98.4 94.8) (width 0.2) (layer "B.Cu") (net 6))
 (segment (start 99.701471 91.9) (end 100.2 91.9) (width 0.2) (layer "B.Cu") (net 6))
 (segment (start 98.4 94.8) (end 98.4 94.55) (width 0.2) (layer "B.Cu") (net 6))
 (segment (start 100.55 92.25) (end 100.55 93.6) (width 0.2) (layer "B.Cu") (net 6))
 (segment (start 100.2 91.9) (end 100.55 92.25) (width 0.2) (layer "B.Cu") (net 6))
 (segment (start 96.934314 95.55) (end 97.65 95.55) (width 0.2) (layer "B.Cu") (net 6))
 (segment (start 95.692157 96.792157) (end 96.934314 95.55) (width 0.2) (layer "B.Cu") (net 6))
 (segment (start 99.35 92.251471) (end 99.701471 91.9) (width 0.2) (layer "B.Cu") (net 6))
 (segment (start 98.4 94.55) (end 99.35 93.6) (width 0.2) (layer "B.Cu") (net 6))
 (segment (start 94.042157 96.792157) (end 95.692157 96.792157) (width 0.2) (layer "B.Cu") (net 6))
 (segment (start 94 96.75) (end 94.042157 96.792157) (width 0.2) (layer "B.Cu") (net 6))
 (segment (start 99.35 93.6) (end 99.35 92.251471) (width 0.2) (layer "B.Cu") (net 6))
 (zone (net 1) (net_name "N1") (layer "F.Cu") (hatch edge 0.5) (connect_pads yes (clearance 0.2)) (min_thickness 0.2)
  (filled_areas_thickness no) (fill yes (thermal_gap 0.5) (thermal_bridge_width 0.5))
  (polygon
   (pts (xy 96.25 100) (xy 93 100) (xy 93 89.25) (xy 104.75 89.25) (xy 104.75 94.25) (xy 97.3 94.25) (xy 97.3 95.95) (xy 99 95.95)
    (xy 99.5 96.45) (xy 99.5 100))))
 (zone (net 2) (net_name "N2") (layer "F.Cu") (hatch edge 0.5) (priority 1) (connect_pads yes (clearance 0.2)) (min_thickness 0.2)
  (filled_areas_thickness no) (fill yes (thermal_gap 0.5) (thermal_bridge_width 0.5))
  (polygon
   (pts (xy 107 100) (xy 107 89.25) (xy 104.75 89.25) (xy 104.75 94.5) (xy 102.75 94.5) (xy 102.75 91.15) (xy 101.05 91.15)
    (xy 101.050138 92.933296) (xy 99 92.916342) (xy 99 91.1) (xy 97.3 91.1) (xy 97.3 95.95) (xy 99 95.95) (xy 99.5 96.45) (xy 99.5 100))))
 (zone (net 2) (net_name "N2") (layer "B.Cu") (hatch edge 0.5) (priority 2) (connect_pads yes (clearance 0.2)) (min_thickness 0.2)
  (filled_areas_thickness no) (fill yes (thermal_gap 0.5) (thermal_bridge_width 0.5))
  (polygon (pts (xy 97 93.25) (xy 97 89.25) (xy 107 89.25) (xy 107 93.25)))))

